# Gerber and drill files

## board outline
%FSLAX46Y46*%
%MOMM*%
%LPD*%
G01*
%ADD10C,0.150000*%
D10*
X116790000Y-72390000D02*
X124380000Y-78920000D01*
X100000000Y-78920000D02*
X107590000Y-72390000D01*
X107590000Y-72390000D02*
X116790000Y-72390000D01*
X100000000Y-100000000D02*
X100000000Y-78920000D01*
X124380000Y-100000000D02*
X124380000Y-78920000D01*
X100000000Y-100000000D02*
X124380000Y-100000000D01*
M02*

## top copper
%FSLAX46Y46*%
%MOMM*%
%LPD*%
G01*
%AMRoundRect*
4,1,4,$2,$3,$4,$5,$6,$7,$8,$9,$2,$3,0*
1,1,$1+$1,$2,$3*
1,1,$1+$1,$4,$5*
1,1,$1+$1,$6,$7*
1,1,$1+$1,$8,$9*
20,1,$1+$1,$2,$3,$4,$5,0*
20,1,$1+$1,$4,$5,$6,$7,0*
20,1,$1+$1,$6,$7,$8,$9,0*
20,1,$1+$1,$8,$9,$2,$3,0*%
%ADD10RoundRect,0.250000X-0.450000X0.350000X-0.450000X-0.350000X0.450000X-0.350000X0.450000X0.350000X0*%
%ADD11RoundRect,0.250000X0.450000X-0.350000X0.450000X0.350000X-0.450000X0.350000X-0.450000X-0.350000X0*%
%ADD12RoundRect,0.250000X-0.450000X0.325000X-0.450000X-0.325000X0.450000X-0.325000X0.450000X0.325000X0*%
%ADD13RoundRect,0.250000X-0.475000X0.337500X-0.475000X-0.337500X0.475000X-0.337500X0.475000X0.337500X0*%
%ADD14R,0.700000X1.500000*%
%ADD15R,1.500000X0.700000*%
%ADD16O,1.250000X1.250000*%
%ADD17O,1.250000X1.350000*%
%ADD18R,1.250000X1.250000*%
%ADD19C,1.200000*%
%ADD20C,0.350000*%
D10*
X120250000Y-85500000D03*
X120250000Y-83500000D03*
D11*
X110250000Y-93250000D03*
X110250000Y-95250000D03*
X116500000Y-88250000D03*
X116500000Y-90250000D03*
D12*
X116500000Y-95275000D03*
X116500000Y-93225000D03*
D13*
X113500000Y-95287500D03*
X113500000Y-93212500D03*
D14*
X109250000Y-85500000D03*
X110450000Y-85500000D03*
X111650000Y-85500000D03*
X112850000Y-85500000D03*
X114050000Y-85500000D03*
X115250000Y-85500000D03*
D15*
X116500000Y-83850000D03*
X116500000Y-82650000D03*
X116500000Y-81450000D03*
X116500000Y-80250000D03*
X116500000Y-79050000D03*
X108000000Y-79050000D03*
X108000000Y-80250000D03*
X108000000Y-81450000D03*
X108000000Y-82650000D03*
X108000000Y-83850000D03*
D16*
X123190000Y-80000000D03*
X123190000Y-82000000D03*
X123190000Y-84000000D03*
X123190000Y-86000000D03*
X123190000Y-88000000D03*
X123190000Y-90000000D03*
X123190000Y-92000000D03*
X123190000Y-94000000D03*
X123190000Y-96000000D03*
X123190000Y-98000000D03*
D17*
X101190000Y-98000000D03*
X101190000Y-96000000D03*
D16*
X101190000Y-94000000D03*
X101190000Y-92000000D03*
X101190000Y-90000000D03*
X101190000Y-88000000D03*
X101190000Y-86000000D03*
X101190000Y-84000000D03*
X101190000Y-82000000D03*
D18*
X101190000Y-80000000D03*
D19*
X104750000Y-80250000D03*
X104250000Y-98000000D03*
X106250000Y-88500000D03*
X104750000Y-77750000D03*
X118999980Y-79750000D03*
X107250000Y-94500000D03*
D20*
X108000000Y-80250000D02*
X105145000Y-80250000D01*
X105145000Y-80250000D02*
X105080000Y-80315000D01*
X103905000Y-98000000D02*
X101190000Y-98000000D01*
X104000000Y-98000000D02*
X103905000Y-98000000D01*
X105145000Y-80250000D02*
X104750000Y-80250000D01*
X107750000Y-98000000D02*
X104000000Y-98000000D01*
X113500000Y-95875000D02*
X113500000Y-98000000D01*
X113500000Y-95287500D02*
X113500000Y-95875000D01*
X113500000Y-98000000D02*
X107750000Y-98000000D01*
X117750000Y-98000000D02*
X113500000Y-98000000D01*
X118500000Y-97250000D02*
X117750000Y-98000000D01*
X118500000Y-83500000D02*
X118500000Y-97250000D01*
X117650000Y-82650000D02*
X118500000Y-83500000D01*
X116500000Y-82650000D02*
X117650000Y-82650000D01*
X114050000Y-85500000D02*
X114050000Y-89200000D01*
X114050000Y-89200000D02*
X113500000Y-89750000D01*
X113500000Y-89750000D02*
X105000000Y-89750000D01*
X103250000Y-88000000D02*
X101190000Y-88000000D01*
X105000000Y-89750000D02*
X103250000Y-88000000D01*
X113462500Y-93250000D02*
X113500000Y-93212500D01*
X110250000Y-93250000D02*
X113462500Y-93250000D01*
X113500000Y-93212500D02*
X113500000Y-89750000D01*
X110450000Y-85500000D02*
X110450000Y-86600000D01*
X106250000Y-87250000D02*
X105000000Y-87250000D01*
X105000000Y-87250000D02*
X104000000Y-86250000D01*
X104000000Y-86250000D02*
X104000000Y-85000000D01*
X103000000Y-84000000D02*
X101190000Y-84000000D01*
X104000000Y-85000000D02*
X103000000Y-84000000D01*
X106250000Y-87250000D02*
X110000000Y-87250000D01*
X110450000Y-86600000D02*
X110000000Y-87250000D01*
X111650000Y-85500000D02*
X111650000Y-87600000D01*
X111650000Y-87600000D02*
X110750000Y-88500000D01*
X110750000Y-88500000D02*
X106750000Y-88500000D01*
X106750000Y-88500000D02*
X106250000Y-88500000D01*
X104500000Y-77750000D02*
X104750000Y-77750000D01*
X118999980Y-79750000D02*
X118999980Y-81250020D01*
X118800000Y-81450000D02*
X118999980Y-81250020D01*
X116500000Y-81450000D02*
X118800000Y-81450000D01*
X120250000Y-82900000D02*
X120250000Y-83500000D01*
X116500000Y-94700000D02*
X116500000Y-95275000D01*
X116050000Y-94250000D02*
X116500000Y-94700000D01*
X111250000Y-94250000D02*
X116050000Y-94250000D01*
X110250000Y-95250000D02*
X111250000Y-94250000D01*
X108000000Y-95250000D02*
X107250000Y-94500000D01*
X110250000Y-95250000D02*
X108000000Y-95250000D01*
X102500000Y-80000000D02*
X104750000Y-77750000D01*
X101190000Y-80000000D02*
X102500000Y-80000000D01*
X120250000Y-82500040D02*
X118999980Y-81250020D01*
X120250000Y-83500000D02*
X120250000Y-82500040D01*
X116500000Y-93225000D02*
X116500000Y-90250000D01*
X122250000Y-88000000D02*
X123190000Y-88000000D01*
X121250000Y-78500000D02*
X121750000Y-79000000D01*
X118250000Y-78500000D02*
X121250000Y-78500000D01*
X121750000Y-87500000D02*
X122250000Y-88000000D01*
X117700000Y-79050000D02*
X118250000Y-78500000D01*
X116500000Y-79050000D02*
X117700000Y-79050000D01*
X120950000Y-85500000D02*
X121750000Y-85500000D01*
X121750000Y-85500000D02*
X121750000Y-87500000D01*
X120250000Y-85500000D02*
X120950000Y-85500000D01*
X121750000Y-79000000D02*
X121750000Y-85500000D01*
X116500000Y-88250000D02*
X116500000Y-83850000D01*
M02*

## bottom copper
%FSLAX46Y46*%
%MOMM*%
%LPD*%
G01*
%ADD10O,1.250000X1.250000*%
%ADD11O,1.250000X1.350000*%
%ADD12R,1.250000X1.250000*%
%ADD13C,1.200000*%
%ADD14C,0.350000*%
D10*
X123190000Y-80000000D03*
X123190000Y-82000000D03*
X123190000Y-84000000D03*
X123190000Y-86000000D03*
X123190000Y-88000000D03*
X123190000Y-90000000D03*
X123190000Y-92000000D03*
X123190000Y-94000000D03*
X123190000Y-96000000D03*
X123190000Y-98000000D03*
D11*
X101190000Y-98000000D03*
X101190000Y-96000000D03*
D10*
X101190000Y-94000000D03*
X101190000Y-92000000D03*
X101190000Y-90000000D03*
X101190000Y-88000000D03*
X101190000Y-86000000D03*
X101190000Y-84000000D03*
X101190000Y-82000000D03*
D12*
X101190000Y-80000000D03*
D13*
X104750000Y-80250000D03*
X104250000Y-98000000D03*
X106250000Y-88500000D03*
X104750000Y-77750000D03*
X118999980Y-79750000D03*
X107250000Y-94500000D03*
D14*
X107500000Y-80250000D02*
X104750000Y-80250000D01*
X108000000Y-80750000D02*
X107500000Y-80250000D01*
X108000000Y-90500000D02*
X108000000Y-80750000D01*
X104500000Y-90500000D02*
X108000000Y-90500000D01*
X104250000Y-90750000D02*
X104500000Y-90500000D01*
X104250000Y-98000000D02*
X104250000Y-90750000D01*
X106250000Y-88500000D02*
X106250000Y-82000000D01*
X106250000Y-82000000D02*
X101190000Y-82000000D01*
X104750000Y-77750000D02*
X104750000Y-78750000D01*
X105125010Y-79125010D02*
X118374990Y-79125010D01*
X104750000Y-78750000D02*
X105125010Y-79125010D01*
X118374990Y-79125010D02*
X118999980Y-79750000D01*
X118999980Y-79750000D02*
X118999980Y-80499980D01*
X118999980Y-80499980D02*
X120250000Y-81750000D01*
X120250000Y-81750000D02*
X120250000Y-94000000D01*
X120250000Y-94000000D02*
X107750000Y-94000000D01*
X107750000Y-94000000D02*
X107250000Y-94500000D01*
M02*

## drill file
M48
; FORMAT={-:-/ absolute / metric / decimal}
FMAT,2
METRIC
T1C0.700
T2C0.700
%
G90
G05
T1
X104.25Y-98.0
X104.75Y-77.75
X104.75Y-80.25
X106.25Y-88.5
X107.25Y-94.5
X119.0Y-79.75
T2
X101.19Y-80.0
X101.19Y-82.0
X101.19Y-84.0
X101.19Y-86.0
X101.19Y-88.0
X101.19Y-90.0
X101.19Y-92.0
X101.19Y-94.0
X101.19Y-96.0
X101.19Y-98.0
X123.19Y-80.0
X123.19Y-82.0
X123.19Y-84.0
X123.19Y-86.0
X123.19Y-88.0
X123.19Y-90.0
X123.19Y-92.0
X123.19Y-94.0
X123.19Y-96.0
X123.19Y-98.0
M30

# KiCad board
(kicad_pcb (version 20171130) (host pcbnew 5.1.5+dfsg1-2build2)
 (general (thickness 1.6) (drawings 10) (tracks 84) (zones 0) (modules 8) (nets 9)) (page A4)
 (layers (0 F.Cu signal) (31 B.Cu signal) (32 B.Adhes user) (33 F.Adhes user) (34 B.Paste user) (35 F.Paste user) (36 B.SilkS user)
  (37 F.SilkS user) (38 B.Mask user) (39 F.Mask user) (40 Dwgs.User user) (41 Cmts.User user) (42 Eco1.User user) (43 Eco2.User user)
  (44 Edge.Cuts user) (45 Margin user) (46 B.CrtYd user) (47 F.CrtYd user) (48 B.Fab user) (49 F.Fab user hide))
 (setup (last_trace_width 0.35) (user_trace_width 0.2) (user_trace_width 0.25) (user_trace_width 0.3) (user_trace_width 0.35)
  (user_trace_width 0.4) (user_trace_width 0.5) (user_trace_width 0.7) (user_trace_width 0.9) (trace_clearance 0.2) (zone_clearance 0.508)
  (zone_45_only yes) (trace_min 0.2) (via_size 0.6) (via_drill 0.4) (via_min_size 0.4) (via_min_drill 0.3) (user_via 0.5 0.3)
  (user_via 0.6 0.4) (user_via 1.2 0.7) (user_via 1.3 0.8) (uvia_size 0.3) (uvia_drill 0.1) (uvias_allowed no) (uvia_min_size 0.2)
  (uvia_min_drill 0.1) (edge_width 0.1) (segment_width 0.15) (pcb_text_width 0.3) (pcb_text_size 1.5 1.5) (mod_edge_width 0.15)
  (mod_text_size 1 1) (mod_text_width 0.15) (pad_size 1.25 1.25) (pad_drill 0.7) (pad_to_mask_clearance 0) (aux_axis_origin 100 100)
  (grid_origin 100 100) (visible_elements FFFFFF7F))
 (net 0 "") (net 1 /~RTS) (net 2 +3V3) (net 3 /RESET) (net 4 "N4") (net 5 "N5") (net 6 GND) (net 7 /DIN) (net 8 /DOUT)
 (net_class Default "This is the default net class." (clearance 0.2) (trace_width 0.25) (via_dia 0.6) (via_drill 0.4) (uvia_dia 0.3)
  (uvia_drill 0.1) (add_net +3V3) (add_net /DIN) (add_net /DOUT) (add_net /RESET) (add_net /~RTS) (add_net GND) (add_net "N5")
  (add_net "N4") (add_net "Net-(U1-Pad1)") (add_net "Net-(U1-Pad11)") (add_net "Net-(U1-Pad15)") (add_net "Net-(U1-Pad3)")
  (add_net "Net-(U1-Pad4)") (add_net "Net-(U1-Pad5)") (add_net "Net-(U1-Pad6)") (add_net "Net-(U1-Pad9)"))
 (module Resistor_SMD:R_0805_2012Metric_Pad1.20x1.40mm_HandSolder (layer F.Cu) (at 120.25 84.5 270)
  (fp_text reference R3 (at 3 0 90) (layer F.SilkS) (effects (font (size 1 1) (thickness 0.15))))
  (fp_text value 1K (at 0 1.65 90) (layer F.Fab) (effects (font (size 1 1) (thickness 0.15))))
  (pad 2 smd roundrect (at 1 0 270) (size 1.2 1.4) (layers F.Cu F.Paste F.Mask) (roundrect_rratio 0.208333) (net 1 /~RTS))
  (pad 1 smd roundrect (at -1 0 270) (size 1.2 1.4) (layers F.Cu F.Paste F.Mask) (roundrect_rratio 0.208333) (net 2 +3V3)))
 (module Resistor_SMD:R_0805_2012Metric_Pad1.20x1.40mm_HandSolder (layer F.Cu) (at 110.25 94.25 90)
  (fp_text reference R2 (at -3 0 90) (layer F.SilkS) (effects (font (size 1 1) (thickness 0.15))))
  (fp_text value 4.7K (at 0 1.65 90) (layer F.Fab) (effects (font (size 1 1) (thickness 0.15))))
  (pad 2 smd roundrect (at 1 0 90) (size 1.2 1.4) (layers F.Cu F.Paste F.Mask) (roundrect_rratio 0.208333) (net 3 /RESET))
  (pad 1 smd roundrect (at -1 0 90) (size 1.2 1.4) (layers F.Cu F.Paste F.Mask) (roundrect_rratio 0.208333) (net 2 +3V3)))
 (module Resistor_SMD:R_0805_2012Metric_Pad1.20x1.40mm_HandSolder (layer F.Cu) (at 116.5 89.25 90)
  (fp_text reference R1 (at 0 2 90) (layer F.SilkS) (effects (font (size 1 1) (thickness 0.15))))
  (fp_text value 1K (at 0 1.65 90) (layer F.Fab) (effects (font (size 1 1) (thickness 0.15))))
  (pad 2 smd roundrect (at 1 0 90) (size 1.2 1.4) (layers F.Cu F.Paste F.Mask) (roundrect_rratio 0.208333) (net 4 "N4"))
  (pad 1 smd roundrect (at -1 0 90) (size 1.2 1.4) (layers F.Cu F.Paste F.Mask) (roundrect_rratio 0.208333) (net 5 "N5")))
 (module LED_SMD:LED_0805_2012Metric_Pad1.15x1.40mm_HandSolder (layer F.Cu) (at 116.5 94.25 270)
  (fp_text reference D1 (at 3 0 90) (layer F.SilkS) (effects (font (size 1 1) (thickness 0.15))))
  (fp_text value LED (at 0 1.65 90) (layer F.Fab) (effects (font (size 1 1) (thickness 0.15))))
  (pad 2 smd roundrect (at 1.025 0 270) (size 1.15 1.4) (layers F.Cu F.Paste F.Mask) (roundrect_rratio 0.217391) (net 2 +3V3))
  (pad 1 smd roundrect (at -1.025 0 270) (size 1.15 1.4) (layers F.Cu F.Paste F.Mask) (roundrect_rratio 0.217391) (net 5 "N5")))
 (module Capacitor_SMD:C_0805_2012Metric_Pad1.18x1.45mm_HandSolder (layer F.Cu) (at 113.5 94.25 270)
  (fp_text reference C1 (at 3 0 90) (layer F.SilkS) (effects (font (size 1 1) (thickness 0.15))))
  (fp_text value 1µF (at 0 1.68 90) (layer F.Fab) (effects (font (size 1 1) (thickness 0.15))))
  (pad 2 smd roundrect (at 1.0375 0 270) (size 1.175 1.45) (layers F.Cu F.Paste F.Mask) (roundrect_rratio 0.212766) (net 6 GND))
  (pad 1 smd roundrect (at -1.0375 0 270) (size 1.175 1.45) (layers F.Cu F.Paste F.Mask) (roundrect_rratio 0.212766) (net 3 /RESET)))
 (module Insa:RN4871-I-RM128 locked (layer F.Cu) (at 107.75 85.75)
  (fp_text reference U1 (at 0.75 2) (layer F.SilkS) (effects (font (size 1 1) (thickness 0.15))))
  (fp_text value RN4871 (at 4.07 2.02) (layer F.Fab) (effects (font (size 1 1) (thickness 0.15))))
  (pad 6 smd rect (at 1.5 -0.25 90) (size 1.5 0.7) (layers F.Cu F.Paste F.Mask))
  (pad 7 smd rect (at 2.7 -0.25 90) (size 1.5 0.7) (layers F.Cu F.Paste F.Mask) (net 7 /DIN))
  (pad 8 smd rect (at 3.9 -0.25 90) (size 1.5 0.7) (layers F.Cu F.Paste F.Mask) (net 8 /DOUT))
  (pad 9 smd rect (at 5.1 -0.25 90) (size 1.5 0.7) (layers F.Cu F.Paste F.Mask))
  (pad 10 smd rect (at 6.3 -0.25 90) (size 1.5 0.7) (layers F.Cu F.Paste F.Mask) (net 3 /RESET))
  (pad 11 smd rect (at 7.5 -0.25 90) (size 1.5 0.7) (layers F.Cu F.Paste F.Mask))
  (pad 12 smd rect (at 8.75 -1.9) (size 1.5 0.7) (layers F.Cu F.Paste F.Mask) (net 4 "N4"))
  (pad 13 smd rect (at 8.75 -3.1) (size 1.5 0.7) (layers F.Cu F.Paste F.Mask) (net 6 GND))
  (pad 14 smd rect (at 8.75 -4.3) (size 1.5 0.7) (layers F.Cu F.Paste F.Mask) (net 2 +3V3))
  (pad 15 smd rect (at 8.75 -5.5) (size 1.5 0.7) (layers F.Cu F.Paste F.Mask))
  (pad 16 smd rect (at 8.75 -6.7) (size 1.5 0.7) (layers F.Cu F.Paste F.Mask) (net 1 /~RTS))
  (pad 1 smd rect (at 0.25 -6.7) (size 1.5 0.7) (layers F.Cu F.Paste F.Mask))
  (pad 2 smd rect (at 0.25 -5.5) (size 1.5 0.7) (layers F.Cu F.Paste F.Mask) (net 6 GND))
  (pad 3 smd rect (at 0.25 -4.3) (size 1.5 0.7) (layers F.Cu F.Paste F.Mask))
  (pad 4 smd rect (at 0.25 -3.1) (size 1.5 0.7) (layers F.Cu F.Paste F.Mask))
  (pad 5 smd rect (at 0.25 -1.9) (size 1.5 0.7) (layers F.Cu F.Paste F.Mask)))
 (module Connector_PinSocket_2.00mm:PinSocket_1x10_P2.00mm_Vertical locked (layer B.Cu) (at 123.19 98)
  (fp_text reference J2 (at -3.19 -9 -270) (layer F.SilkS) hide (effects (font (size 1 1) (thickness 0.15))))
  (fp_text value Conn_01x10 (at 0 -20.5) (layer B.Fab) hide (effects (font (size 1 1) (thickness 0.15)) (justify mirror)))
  (pad 10 thru_hole oval (at 0 -18) (size 1.25 1.25) (drill 0.7) (layers *.Cu *.Mask))
  (pad 9 thru_hole oval (at 0 -16) (size 1.25 1.25) (drill 0.7) (layers *.Cu *.Mask))
  (pad 8 thru_hole oval (at 0 -14) (size 1.25 1.25) (drill 0.7) (layers *.Cu *.Mask))
  (pad 7 thru_hole oval (at 0 -12) (size 1.25 1.25) (drill 0.7) (layers *.Cu *.Mask))
  (pad 6 thru_hole oval (at 0 -10) (size 1.25 1.25) (drill 0.7) (layers *.Cu *.Mask) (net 1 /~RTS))
  (pad 5 thru_hole oval (at 0 -8) (size 1.25 1.25) (drill 0.7) (layers *.Cu *.Mask))
  (pad 4 thru_hole oval (at 0 -6) (size 1.25 1.25) (drill 0.7) (layers *.Cu *.Mask))
  (pad 3 thru_hole oval (at 0 -4) (size 1.25 1.25) (drill 0.7) (layers *.Cu *.Mask))
  (pad 2 thru_hole oval (at 0 -2) (size 1.25 1.25) (drill 0.7) (layers *.Cu *.Mask))
  (pad 1 thru_hole oval (at 0 0) (size 1.25 1.25) (drill 0.7) (layers *.Cu *.Mask)))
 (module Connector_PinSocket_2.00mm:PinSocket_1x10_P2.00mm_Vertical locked (layer B.Cu) (at 101.19 80 180)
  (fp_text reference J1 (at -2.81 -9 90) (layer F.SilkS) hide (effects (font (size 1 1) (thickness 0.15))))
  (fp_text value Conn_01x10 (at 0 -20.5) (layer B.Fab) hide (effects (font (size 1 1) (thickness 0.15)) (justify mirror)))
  (pad 10 thru_hole oval (at 0 -18 180) (size 1.25 1.35) (drill 0.7) (layers *.Cu *.Mask) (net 6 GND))
  (pad 9 thru_hole oval (at 0 -16 180) (size 1.25 1.35) (drill 0.7) (layers *.Cu *.Mask))
  (pad 8 thru_hole oval (at 0 -14 180) (size 1.25 1.25) (drill 0.7) (layers *.Cu *.Mask))
  (pad 7 thru_hole oval (at 0 -12 180) (size 1.25 1.25) (drill 0.7) (layers *.Cu *.Mask))
  (pad 6 thru_hole oval (at 0 -10 180) (size 1.25 1.25) (drill 0.7) (layers *.Cu *.Mask))
  (pad 5 thru_hole oval (at 0 -8 180) (size 1.25 1.25) (drill 0.7) (layers *.Cu *.Mask) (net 3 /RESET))
  (pad 4 thru_hole oval (at 0 -6 180) (size 1.25 1.25) (drill 0.7) (layers *.Cu *.Mask))
  (pad 3 thru_hole oval (at 0 -4 180) (size 1.25 1.25) (drill 0.7) (layers *.Cu *.Mask) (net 7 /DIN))
  (pad 2 thru_hole oval (at 0 -2 180) (size 1.25 1.25) (drill 0.7) (layers *.Cu *.Mask) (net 8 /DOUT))
  (pad 1 thru_hole rect (at 0 0 180) (size 1.25 1.25) (drill 0.7) (layers *.Cu *.Mask) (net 2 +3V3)))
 (gr_line (start 116.79 72.39) (end 124.38 78.92) (layer Edge.Cuts) (width 0.15))
 (gr_line (start 100 78.92) (end 107.59 72.39) (layer Edge.Cuts) (width 0.15))
 (gr_line (start 107.59 72.39) (end 116.79 72.39) (layer Edge.Cuts) (width 0.15))
 (gr_line (start 100 100) (end 100 78.92) (layer Edge.Cuts) (width 0.15))
 (gr_line (start 124.38 100) (end 124.38 78.92) (layer Edge.Cuts) (width 0.15))
 (gr_line (start 100 100) (end 124.38 100) (layer Edge.Cuts) (width 0.15))
 (segment (start 108 80.25) (end 105.145 80.25) (width 0.35) (layer F.Cu) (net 6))
 (segment (start 105.145 80.25) (end 105.08 80.315) (width 0.35) (layer F.Cu) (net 6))
 (segment (start 103.905 98) (end 101.19 98) (width 0.35) (layer F.Cu) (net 6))
 (segment (start 104 98) (end 103.905 98) (width 0.35) (layer F.Cu) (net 6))
 (via (at 104.75 80.25) (size 1.2) (drill 0.7) (layers F.Cu B.Cu) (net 6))
 (segment (start 105.145 80.25) (end 104.75 80.25) (width 0.35) (layer F.Cu) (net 6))
 (via (at 104.25 98) (size 1.2) (drill 0.7) (layers F.Cu B.Cu) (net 6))
 (segment (start 107.75 98) (end 104 98) (width 0.35) (layer F.Cu) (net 6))
 (segment (start 113.5 95.875) (end 113.5 98) (width 0.35) (layer F.Cu) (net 6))
 (segment (start 113.5 95.2875) (end 113.5 95.875) (width 0.35) (layer F.Cu) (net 6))
 (segment (start 113.5 98) (end 107.75 98) (width 0.35) (layer F.Cu) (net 6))
 (segment (start 107.5 80.25) (end 104.75 80.25) (width 0.35) (layer B.Cu) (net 6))
 (segment (start 108 80.75) (end 107.5 80.25) (width 0.35) (layer B.Cu) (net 6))
 (segment (start 108 90.5) (end 108 80.75) (width 0.35) (layer B.Cu) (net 6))
 (segment (start 104.5 90.5) (end 108 90.5) (width 0.35) (layer B.Cu) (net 6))
 (segment (start 104.25 90.75) (end 104.5 90.5) (width 0.35) (layer B.Cu) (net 6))
 (segment (start 104.25 98) (end 104.25 90.75) (width 0.35) (layer B.Cu) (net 6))
 (segment (start 117.75 98) (end 113.5 98) (width 0.35) (layer F.Cu) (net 6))
 (segment (start 118.5 97.25) (end 117.75 98) (width 0.35) (layer F.Cu) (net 6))
 (segment (start 118.5 83.5) (end 118.5 97.25) (width 0.35) (layer F.Cu) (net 6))
 (segment (start 117.65 82.65) (end 118.5 83.5) (width 0.35) (layer F.Cu) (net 6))
 (segment (start 116.5 82.65) (end 117.65 82.65) (width 0.35) (layer F.Cu) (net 6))
 (segment (start 114.05 85.5) (end 114.05 89.2) (width 0.35) (layer F.Cu) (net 3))
 (segment (start 114.05 89.2) (end 113.5 89.75) (width 0.35) (layer F.Cu) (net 3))
 (segment (start 113.5 89.75) (end 105 89.75) (width 0.35) (layer F.Cu) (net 3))
 (segment (start 103.25 88) (end 101.19 88) (width 0.35) (layer F.Cu) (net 3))
 (segment (start 105 89.75) (end 103.25 88) (width 0.35) (layer F.Cu) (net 3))
 (segment (start 113.4625 93.25) (end 113.5 93.2125) (width 0.35) (layer F.Cu) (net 3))
 (segment (start 110.25 93.25) (end 113.4625 93.25) (width 0.35) (layer F.Cu) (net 3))
 (segment (start 113.5 93.2125) (end 113.5 89.75) (width 0.35) (layer F.Cu) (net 3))
 (segment (start 110.45 85.5) (end 110.45 86.6) (width 0.35) (layer F.Cu) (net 7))
 (segment (start 106.25 87.25) (end 105 87.25) (width 0.35) (layer F.Cu) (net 7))
 (segment (start 105 87.25) (end 104 86.25) (width 0.35) (layer F.Cu) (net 7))
 (segment (start 104 86.25) (end 104 85) (width 0.35) (layer F.Cu) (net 7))
 (segment (start 103 84) (end 101.19 84) (width 0.35) (layer F.Cu) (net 7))
 (segment (start 104 85) (end 103 84) (width 0.35) (layer F.Cu) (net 7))
 (segment (start 106.25 87.25) (end 110 87.25) (width 0.35) (layer F.Cu) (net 7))
 (segment (start 110.45 86.6) (end 110 87.25) (width 0.35) (layer F.Cu) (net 7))
 (segment (start 111.65 85.5) (end 111.65 87.6) (width 0.35) (layer F.Cu) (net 8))
 (segment (start 111.65 87.6) (end 110.75 88.5) (width 0.35) (layer F.Cu) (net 8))
 (segment (start 110.75 88.5) (end 106.75 88.5) (width 0.35) (layer F.Cu) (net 8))
 (via (at 106.25 88.5) (size 1.2) (drill 0.7) (layers F.Cu B.Cu) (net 8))
 (segment (start 106.75 88.5) (end 106.25 88.5) (width 0.35) (layer F.Cu) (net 8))
 (segment (start 106.25 88.5) (end 106.25 82) (width 0.35) (layer B.Cu) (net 8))
 (segment (start 106.25 82) (end 101.19 82) (width 0.35) (layer B.Cu) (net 8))
 (via (at 104.75 77.75) (size 1.2) (drill 0.7) (layers F.Cu B.Cu) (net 2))
 (segment (start 104.5 77.75) (end 104.75 77.75) (width 0.35) (layer F.Cu) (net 2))
 (segment (start 104.75 77.75) (end 104.75 78.75) (width 0.35) (layer B.Cu) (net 2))
 (segment (start 105.12501 79.12501) (end 118.37499 79.12501) (width 0.35) (layer B.Cu) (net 2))
 (segment (start 104.75 78.75) (end 105.12501 79.12501) (width 0.35) (layer B.Cu) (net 2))
 (segment (start 118.37499 79.12501) (end 118.99998 79.75) (width 0.35) (layer B.Cu) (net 2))
 (via (at 118.99998 79.75) (size 1.2) (drill 0.7) (layers F.Cu B.Cu) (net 2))
 (segment (start 118.99998 79.75) (end 118.99998 81.25002) (width 0.35) (layer F.Cu) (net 2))
 (segment (start 118.8 81.45) (end 118.99998 81.25002) (width 0.35) (layer F.Cu) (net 2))
 (segment (start 116.5 81.45) (end 118.8 81.45) (width 0.35) (layer F.Cu) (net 2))
 (segment (start 120.25 82.9) (end 120.25 83.5) (width 0.35) (layer F.Cu) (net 2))
 (segment (start 116.5 94.7) (end 116.5 95.275) (width 0.35) (layer F.Cu) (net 2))
 (segment (start 116.05 94.25) (end 116.5 94.7) (width 0.35) (layer F.Cu) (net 2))
 (segment (start 111.25 94.25) (end 116.05 94.25) (width 0.35) (layer F.Cu) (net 2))
 (segment (start 110.25 95.25) (end 111.25 94.25) (width 0.35) (layer F.Cu) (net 2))
 (segment (start 118.99998 79.75) (end 118.99998 80.49998) (width 0.35) (layer B.Cu) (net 2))
 (segment (start 118.99998 80.49998) (end 120.25 81.75) (width 0.35) (layer B.Cu) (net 2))
 (segment (start 120.25 81.75) (end 120.25 94) (width 0.35) (layer B.Cu) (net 2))
 (segment (start 120.25 94) (end 107.75 94) (width 0.35) (layer B.Cu) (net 2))
 (via (at 107.25 94.5) (size 1.2) (drill 0.7) (layers F.Cu B.Cu) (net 2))
 (segment (start 107.75 94) (end 107.25 94.5) (width 0.35) (layer B.Cu) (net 2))
 (segment (start 108 95.25) (end 107.25 94.5) (width 0.35) (layer F.Cu) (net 2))
 (segment (start 110.25 95.25) (end 108 95.25) (width 0.35) (layer F.Cu) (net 2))
 (segment (start 102.5 80) (end 104.75 77.75) (width 0.35) (layer F.Cu) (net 2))
 (segment (start 101.19 80) (end 102.5 80) (width 0.35) (layer F.Cu) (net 2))
 (segment (start 120.25 82.50004) (end 118.99998 81.25002) (width 0.35) (layer F.Cu) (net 2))
 (segment (start 120.25 83.5) (end 120.25 82.50004) (width 0.35) (layer F.Cu) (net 2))
 (segment (start 116.5 93.225) (end 116.5 90.25) (width 0.35) (layer F.Cu) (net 5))
 (segment (start 122.25 88) (end 123.19 88) (width 0.35) (layer F.Cu) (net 1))
 (segment (start 121.25 78.5) (end 121.75 79) (width 0.35) (layer F.Cu) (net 1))
 (segment (start 118.25 78.5) (end 121.25 78.5) (width 0.35) (layer F.Cu) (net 1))
 (segment (start 121.75 87.5) (end 122.25 88) (width 0.35) (layer F.Cu) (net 1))
 (segment (start 117.7 79.05) (end 118.25 78.5) (width 0.35) (layer F.Cu) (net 1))
 (segment (start 116.5 79.05) (end 117.7 79.05) (width 0.35) (layer F.Cu) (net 1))
 (segment (start 120.95 85.5) (end 121.75 85.5) (width 0.35) (layer F.Cu) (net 1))
 (segment (start 121.75 85.5) (end 121.75 87.5) (width 0.35) (layer F.Cu) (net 1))
 (segment (start 120.25 85.5) (end 120.95 85.5) (width 0.35) (layer F.Cu) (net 1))
 (segment (start 121.75 79) (end 121.75 85.5) (width 0.35) (layer F.Cu) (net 1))
 (segment (start 116.5 88.25) (end 116.5 83.85) (width 0.35) (layer F.Cu) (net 4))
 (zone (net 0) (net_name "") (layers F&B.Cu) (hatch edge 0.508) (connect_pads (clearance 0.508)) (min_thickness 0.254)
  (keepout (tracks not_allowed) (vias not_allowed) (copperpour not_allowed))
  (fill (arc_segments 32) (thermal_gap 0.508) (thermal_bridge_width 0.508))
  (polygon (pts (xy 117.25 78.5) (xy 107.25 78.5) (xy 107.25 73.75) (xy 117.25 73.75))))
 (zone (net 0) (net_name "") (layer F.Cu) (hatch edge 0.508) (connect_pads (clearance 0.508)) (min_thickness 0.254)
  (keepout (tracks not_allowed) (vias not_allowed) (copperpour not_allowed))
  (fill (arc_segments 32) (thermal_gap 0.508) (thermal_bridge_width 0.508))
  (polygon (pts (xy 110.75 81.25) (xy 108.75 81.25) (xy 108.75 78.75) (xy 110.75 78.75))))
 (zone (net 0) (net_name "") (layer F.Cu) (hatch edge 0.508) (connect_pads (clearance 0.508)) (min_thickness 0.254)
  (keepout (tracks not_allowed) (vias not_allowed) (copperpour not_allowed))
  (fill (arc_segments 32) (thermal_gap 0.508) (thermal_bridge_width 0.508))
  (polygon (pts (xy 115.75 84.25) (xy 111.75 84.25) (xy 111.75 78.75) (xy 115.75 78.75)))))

